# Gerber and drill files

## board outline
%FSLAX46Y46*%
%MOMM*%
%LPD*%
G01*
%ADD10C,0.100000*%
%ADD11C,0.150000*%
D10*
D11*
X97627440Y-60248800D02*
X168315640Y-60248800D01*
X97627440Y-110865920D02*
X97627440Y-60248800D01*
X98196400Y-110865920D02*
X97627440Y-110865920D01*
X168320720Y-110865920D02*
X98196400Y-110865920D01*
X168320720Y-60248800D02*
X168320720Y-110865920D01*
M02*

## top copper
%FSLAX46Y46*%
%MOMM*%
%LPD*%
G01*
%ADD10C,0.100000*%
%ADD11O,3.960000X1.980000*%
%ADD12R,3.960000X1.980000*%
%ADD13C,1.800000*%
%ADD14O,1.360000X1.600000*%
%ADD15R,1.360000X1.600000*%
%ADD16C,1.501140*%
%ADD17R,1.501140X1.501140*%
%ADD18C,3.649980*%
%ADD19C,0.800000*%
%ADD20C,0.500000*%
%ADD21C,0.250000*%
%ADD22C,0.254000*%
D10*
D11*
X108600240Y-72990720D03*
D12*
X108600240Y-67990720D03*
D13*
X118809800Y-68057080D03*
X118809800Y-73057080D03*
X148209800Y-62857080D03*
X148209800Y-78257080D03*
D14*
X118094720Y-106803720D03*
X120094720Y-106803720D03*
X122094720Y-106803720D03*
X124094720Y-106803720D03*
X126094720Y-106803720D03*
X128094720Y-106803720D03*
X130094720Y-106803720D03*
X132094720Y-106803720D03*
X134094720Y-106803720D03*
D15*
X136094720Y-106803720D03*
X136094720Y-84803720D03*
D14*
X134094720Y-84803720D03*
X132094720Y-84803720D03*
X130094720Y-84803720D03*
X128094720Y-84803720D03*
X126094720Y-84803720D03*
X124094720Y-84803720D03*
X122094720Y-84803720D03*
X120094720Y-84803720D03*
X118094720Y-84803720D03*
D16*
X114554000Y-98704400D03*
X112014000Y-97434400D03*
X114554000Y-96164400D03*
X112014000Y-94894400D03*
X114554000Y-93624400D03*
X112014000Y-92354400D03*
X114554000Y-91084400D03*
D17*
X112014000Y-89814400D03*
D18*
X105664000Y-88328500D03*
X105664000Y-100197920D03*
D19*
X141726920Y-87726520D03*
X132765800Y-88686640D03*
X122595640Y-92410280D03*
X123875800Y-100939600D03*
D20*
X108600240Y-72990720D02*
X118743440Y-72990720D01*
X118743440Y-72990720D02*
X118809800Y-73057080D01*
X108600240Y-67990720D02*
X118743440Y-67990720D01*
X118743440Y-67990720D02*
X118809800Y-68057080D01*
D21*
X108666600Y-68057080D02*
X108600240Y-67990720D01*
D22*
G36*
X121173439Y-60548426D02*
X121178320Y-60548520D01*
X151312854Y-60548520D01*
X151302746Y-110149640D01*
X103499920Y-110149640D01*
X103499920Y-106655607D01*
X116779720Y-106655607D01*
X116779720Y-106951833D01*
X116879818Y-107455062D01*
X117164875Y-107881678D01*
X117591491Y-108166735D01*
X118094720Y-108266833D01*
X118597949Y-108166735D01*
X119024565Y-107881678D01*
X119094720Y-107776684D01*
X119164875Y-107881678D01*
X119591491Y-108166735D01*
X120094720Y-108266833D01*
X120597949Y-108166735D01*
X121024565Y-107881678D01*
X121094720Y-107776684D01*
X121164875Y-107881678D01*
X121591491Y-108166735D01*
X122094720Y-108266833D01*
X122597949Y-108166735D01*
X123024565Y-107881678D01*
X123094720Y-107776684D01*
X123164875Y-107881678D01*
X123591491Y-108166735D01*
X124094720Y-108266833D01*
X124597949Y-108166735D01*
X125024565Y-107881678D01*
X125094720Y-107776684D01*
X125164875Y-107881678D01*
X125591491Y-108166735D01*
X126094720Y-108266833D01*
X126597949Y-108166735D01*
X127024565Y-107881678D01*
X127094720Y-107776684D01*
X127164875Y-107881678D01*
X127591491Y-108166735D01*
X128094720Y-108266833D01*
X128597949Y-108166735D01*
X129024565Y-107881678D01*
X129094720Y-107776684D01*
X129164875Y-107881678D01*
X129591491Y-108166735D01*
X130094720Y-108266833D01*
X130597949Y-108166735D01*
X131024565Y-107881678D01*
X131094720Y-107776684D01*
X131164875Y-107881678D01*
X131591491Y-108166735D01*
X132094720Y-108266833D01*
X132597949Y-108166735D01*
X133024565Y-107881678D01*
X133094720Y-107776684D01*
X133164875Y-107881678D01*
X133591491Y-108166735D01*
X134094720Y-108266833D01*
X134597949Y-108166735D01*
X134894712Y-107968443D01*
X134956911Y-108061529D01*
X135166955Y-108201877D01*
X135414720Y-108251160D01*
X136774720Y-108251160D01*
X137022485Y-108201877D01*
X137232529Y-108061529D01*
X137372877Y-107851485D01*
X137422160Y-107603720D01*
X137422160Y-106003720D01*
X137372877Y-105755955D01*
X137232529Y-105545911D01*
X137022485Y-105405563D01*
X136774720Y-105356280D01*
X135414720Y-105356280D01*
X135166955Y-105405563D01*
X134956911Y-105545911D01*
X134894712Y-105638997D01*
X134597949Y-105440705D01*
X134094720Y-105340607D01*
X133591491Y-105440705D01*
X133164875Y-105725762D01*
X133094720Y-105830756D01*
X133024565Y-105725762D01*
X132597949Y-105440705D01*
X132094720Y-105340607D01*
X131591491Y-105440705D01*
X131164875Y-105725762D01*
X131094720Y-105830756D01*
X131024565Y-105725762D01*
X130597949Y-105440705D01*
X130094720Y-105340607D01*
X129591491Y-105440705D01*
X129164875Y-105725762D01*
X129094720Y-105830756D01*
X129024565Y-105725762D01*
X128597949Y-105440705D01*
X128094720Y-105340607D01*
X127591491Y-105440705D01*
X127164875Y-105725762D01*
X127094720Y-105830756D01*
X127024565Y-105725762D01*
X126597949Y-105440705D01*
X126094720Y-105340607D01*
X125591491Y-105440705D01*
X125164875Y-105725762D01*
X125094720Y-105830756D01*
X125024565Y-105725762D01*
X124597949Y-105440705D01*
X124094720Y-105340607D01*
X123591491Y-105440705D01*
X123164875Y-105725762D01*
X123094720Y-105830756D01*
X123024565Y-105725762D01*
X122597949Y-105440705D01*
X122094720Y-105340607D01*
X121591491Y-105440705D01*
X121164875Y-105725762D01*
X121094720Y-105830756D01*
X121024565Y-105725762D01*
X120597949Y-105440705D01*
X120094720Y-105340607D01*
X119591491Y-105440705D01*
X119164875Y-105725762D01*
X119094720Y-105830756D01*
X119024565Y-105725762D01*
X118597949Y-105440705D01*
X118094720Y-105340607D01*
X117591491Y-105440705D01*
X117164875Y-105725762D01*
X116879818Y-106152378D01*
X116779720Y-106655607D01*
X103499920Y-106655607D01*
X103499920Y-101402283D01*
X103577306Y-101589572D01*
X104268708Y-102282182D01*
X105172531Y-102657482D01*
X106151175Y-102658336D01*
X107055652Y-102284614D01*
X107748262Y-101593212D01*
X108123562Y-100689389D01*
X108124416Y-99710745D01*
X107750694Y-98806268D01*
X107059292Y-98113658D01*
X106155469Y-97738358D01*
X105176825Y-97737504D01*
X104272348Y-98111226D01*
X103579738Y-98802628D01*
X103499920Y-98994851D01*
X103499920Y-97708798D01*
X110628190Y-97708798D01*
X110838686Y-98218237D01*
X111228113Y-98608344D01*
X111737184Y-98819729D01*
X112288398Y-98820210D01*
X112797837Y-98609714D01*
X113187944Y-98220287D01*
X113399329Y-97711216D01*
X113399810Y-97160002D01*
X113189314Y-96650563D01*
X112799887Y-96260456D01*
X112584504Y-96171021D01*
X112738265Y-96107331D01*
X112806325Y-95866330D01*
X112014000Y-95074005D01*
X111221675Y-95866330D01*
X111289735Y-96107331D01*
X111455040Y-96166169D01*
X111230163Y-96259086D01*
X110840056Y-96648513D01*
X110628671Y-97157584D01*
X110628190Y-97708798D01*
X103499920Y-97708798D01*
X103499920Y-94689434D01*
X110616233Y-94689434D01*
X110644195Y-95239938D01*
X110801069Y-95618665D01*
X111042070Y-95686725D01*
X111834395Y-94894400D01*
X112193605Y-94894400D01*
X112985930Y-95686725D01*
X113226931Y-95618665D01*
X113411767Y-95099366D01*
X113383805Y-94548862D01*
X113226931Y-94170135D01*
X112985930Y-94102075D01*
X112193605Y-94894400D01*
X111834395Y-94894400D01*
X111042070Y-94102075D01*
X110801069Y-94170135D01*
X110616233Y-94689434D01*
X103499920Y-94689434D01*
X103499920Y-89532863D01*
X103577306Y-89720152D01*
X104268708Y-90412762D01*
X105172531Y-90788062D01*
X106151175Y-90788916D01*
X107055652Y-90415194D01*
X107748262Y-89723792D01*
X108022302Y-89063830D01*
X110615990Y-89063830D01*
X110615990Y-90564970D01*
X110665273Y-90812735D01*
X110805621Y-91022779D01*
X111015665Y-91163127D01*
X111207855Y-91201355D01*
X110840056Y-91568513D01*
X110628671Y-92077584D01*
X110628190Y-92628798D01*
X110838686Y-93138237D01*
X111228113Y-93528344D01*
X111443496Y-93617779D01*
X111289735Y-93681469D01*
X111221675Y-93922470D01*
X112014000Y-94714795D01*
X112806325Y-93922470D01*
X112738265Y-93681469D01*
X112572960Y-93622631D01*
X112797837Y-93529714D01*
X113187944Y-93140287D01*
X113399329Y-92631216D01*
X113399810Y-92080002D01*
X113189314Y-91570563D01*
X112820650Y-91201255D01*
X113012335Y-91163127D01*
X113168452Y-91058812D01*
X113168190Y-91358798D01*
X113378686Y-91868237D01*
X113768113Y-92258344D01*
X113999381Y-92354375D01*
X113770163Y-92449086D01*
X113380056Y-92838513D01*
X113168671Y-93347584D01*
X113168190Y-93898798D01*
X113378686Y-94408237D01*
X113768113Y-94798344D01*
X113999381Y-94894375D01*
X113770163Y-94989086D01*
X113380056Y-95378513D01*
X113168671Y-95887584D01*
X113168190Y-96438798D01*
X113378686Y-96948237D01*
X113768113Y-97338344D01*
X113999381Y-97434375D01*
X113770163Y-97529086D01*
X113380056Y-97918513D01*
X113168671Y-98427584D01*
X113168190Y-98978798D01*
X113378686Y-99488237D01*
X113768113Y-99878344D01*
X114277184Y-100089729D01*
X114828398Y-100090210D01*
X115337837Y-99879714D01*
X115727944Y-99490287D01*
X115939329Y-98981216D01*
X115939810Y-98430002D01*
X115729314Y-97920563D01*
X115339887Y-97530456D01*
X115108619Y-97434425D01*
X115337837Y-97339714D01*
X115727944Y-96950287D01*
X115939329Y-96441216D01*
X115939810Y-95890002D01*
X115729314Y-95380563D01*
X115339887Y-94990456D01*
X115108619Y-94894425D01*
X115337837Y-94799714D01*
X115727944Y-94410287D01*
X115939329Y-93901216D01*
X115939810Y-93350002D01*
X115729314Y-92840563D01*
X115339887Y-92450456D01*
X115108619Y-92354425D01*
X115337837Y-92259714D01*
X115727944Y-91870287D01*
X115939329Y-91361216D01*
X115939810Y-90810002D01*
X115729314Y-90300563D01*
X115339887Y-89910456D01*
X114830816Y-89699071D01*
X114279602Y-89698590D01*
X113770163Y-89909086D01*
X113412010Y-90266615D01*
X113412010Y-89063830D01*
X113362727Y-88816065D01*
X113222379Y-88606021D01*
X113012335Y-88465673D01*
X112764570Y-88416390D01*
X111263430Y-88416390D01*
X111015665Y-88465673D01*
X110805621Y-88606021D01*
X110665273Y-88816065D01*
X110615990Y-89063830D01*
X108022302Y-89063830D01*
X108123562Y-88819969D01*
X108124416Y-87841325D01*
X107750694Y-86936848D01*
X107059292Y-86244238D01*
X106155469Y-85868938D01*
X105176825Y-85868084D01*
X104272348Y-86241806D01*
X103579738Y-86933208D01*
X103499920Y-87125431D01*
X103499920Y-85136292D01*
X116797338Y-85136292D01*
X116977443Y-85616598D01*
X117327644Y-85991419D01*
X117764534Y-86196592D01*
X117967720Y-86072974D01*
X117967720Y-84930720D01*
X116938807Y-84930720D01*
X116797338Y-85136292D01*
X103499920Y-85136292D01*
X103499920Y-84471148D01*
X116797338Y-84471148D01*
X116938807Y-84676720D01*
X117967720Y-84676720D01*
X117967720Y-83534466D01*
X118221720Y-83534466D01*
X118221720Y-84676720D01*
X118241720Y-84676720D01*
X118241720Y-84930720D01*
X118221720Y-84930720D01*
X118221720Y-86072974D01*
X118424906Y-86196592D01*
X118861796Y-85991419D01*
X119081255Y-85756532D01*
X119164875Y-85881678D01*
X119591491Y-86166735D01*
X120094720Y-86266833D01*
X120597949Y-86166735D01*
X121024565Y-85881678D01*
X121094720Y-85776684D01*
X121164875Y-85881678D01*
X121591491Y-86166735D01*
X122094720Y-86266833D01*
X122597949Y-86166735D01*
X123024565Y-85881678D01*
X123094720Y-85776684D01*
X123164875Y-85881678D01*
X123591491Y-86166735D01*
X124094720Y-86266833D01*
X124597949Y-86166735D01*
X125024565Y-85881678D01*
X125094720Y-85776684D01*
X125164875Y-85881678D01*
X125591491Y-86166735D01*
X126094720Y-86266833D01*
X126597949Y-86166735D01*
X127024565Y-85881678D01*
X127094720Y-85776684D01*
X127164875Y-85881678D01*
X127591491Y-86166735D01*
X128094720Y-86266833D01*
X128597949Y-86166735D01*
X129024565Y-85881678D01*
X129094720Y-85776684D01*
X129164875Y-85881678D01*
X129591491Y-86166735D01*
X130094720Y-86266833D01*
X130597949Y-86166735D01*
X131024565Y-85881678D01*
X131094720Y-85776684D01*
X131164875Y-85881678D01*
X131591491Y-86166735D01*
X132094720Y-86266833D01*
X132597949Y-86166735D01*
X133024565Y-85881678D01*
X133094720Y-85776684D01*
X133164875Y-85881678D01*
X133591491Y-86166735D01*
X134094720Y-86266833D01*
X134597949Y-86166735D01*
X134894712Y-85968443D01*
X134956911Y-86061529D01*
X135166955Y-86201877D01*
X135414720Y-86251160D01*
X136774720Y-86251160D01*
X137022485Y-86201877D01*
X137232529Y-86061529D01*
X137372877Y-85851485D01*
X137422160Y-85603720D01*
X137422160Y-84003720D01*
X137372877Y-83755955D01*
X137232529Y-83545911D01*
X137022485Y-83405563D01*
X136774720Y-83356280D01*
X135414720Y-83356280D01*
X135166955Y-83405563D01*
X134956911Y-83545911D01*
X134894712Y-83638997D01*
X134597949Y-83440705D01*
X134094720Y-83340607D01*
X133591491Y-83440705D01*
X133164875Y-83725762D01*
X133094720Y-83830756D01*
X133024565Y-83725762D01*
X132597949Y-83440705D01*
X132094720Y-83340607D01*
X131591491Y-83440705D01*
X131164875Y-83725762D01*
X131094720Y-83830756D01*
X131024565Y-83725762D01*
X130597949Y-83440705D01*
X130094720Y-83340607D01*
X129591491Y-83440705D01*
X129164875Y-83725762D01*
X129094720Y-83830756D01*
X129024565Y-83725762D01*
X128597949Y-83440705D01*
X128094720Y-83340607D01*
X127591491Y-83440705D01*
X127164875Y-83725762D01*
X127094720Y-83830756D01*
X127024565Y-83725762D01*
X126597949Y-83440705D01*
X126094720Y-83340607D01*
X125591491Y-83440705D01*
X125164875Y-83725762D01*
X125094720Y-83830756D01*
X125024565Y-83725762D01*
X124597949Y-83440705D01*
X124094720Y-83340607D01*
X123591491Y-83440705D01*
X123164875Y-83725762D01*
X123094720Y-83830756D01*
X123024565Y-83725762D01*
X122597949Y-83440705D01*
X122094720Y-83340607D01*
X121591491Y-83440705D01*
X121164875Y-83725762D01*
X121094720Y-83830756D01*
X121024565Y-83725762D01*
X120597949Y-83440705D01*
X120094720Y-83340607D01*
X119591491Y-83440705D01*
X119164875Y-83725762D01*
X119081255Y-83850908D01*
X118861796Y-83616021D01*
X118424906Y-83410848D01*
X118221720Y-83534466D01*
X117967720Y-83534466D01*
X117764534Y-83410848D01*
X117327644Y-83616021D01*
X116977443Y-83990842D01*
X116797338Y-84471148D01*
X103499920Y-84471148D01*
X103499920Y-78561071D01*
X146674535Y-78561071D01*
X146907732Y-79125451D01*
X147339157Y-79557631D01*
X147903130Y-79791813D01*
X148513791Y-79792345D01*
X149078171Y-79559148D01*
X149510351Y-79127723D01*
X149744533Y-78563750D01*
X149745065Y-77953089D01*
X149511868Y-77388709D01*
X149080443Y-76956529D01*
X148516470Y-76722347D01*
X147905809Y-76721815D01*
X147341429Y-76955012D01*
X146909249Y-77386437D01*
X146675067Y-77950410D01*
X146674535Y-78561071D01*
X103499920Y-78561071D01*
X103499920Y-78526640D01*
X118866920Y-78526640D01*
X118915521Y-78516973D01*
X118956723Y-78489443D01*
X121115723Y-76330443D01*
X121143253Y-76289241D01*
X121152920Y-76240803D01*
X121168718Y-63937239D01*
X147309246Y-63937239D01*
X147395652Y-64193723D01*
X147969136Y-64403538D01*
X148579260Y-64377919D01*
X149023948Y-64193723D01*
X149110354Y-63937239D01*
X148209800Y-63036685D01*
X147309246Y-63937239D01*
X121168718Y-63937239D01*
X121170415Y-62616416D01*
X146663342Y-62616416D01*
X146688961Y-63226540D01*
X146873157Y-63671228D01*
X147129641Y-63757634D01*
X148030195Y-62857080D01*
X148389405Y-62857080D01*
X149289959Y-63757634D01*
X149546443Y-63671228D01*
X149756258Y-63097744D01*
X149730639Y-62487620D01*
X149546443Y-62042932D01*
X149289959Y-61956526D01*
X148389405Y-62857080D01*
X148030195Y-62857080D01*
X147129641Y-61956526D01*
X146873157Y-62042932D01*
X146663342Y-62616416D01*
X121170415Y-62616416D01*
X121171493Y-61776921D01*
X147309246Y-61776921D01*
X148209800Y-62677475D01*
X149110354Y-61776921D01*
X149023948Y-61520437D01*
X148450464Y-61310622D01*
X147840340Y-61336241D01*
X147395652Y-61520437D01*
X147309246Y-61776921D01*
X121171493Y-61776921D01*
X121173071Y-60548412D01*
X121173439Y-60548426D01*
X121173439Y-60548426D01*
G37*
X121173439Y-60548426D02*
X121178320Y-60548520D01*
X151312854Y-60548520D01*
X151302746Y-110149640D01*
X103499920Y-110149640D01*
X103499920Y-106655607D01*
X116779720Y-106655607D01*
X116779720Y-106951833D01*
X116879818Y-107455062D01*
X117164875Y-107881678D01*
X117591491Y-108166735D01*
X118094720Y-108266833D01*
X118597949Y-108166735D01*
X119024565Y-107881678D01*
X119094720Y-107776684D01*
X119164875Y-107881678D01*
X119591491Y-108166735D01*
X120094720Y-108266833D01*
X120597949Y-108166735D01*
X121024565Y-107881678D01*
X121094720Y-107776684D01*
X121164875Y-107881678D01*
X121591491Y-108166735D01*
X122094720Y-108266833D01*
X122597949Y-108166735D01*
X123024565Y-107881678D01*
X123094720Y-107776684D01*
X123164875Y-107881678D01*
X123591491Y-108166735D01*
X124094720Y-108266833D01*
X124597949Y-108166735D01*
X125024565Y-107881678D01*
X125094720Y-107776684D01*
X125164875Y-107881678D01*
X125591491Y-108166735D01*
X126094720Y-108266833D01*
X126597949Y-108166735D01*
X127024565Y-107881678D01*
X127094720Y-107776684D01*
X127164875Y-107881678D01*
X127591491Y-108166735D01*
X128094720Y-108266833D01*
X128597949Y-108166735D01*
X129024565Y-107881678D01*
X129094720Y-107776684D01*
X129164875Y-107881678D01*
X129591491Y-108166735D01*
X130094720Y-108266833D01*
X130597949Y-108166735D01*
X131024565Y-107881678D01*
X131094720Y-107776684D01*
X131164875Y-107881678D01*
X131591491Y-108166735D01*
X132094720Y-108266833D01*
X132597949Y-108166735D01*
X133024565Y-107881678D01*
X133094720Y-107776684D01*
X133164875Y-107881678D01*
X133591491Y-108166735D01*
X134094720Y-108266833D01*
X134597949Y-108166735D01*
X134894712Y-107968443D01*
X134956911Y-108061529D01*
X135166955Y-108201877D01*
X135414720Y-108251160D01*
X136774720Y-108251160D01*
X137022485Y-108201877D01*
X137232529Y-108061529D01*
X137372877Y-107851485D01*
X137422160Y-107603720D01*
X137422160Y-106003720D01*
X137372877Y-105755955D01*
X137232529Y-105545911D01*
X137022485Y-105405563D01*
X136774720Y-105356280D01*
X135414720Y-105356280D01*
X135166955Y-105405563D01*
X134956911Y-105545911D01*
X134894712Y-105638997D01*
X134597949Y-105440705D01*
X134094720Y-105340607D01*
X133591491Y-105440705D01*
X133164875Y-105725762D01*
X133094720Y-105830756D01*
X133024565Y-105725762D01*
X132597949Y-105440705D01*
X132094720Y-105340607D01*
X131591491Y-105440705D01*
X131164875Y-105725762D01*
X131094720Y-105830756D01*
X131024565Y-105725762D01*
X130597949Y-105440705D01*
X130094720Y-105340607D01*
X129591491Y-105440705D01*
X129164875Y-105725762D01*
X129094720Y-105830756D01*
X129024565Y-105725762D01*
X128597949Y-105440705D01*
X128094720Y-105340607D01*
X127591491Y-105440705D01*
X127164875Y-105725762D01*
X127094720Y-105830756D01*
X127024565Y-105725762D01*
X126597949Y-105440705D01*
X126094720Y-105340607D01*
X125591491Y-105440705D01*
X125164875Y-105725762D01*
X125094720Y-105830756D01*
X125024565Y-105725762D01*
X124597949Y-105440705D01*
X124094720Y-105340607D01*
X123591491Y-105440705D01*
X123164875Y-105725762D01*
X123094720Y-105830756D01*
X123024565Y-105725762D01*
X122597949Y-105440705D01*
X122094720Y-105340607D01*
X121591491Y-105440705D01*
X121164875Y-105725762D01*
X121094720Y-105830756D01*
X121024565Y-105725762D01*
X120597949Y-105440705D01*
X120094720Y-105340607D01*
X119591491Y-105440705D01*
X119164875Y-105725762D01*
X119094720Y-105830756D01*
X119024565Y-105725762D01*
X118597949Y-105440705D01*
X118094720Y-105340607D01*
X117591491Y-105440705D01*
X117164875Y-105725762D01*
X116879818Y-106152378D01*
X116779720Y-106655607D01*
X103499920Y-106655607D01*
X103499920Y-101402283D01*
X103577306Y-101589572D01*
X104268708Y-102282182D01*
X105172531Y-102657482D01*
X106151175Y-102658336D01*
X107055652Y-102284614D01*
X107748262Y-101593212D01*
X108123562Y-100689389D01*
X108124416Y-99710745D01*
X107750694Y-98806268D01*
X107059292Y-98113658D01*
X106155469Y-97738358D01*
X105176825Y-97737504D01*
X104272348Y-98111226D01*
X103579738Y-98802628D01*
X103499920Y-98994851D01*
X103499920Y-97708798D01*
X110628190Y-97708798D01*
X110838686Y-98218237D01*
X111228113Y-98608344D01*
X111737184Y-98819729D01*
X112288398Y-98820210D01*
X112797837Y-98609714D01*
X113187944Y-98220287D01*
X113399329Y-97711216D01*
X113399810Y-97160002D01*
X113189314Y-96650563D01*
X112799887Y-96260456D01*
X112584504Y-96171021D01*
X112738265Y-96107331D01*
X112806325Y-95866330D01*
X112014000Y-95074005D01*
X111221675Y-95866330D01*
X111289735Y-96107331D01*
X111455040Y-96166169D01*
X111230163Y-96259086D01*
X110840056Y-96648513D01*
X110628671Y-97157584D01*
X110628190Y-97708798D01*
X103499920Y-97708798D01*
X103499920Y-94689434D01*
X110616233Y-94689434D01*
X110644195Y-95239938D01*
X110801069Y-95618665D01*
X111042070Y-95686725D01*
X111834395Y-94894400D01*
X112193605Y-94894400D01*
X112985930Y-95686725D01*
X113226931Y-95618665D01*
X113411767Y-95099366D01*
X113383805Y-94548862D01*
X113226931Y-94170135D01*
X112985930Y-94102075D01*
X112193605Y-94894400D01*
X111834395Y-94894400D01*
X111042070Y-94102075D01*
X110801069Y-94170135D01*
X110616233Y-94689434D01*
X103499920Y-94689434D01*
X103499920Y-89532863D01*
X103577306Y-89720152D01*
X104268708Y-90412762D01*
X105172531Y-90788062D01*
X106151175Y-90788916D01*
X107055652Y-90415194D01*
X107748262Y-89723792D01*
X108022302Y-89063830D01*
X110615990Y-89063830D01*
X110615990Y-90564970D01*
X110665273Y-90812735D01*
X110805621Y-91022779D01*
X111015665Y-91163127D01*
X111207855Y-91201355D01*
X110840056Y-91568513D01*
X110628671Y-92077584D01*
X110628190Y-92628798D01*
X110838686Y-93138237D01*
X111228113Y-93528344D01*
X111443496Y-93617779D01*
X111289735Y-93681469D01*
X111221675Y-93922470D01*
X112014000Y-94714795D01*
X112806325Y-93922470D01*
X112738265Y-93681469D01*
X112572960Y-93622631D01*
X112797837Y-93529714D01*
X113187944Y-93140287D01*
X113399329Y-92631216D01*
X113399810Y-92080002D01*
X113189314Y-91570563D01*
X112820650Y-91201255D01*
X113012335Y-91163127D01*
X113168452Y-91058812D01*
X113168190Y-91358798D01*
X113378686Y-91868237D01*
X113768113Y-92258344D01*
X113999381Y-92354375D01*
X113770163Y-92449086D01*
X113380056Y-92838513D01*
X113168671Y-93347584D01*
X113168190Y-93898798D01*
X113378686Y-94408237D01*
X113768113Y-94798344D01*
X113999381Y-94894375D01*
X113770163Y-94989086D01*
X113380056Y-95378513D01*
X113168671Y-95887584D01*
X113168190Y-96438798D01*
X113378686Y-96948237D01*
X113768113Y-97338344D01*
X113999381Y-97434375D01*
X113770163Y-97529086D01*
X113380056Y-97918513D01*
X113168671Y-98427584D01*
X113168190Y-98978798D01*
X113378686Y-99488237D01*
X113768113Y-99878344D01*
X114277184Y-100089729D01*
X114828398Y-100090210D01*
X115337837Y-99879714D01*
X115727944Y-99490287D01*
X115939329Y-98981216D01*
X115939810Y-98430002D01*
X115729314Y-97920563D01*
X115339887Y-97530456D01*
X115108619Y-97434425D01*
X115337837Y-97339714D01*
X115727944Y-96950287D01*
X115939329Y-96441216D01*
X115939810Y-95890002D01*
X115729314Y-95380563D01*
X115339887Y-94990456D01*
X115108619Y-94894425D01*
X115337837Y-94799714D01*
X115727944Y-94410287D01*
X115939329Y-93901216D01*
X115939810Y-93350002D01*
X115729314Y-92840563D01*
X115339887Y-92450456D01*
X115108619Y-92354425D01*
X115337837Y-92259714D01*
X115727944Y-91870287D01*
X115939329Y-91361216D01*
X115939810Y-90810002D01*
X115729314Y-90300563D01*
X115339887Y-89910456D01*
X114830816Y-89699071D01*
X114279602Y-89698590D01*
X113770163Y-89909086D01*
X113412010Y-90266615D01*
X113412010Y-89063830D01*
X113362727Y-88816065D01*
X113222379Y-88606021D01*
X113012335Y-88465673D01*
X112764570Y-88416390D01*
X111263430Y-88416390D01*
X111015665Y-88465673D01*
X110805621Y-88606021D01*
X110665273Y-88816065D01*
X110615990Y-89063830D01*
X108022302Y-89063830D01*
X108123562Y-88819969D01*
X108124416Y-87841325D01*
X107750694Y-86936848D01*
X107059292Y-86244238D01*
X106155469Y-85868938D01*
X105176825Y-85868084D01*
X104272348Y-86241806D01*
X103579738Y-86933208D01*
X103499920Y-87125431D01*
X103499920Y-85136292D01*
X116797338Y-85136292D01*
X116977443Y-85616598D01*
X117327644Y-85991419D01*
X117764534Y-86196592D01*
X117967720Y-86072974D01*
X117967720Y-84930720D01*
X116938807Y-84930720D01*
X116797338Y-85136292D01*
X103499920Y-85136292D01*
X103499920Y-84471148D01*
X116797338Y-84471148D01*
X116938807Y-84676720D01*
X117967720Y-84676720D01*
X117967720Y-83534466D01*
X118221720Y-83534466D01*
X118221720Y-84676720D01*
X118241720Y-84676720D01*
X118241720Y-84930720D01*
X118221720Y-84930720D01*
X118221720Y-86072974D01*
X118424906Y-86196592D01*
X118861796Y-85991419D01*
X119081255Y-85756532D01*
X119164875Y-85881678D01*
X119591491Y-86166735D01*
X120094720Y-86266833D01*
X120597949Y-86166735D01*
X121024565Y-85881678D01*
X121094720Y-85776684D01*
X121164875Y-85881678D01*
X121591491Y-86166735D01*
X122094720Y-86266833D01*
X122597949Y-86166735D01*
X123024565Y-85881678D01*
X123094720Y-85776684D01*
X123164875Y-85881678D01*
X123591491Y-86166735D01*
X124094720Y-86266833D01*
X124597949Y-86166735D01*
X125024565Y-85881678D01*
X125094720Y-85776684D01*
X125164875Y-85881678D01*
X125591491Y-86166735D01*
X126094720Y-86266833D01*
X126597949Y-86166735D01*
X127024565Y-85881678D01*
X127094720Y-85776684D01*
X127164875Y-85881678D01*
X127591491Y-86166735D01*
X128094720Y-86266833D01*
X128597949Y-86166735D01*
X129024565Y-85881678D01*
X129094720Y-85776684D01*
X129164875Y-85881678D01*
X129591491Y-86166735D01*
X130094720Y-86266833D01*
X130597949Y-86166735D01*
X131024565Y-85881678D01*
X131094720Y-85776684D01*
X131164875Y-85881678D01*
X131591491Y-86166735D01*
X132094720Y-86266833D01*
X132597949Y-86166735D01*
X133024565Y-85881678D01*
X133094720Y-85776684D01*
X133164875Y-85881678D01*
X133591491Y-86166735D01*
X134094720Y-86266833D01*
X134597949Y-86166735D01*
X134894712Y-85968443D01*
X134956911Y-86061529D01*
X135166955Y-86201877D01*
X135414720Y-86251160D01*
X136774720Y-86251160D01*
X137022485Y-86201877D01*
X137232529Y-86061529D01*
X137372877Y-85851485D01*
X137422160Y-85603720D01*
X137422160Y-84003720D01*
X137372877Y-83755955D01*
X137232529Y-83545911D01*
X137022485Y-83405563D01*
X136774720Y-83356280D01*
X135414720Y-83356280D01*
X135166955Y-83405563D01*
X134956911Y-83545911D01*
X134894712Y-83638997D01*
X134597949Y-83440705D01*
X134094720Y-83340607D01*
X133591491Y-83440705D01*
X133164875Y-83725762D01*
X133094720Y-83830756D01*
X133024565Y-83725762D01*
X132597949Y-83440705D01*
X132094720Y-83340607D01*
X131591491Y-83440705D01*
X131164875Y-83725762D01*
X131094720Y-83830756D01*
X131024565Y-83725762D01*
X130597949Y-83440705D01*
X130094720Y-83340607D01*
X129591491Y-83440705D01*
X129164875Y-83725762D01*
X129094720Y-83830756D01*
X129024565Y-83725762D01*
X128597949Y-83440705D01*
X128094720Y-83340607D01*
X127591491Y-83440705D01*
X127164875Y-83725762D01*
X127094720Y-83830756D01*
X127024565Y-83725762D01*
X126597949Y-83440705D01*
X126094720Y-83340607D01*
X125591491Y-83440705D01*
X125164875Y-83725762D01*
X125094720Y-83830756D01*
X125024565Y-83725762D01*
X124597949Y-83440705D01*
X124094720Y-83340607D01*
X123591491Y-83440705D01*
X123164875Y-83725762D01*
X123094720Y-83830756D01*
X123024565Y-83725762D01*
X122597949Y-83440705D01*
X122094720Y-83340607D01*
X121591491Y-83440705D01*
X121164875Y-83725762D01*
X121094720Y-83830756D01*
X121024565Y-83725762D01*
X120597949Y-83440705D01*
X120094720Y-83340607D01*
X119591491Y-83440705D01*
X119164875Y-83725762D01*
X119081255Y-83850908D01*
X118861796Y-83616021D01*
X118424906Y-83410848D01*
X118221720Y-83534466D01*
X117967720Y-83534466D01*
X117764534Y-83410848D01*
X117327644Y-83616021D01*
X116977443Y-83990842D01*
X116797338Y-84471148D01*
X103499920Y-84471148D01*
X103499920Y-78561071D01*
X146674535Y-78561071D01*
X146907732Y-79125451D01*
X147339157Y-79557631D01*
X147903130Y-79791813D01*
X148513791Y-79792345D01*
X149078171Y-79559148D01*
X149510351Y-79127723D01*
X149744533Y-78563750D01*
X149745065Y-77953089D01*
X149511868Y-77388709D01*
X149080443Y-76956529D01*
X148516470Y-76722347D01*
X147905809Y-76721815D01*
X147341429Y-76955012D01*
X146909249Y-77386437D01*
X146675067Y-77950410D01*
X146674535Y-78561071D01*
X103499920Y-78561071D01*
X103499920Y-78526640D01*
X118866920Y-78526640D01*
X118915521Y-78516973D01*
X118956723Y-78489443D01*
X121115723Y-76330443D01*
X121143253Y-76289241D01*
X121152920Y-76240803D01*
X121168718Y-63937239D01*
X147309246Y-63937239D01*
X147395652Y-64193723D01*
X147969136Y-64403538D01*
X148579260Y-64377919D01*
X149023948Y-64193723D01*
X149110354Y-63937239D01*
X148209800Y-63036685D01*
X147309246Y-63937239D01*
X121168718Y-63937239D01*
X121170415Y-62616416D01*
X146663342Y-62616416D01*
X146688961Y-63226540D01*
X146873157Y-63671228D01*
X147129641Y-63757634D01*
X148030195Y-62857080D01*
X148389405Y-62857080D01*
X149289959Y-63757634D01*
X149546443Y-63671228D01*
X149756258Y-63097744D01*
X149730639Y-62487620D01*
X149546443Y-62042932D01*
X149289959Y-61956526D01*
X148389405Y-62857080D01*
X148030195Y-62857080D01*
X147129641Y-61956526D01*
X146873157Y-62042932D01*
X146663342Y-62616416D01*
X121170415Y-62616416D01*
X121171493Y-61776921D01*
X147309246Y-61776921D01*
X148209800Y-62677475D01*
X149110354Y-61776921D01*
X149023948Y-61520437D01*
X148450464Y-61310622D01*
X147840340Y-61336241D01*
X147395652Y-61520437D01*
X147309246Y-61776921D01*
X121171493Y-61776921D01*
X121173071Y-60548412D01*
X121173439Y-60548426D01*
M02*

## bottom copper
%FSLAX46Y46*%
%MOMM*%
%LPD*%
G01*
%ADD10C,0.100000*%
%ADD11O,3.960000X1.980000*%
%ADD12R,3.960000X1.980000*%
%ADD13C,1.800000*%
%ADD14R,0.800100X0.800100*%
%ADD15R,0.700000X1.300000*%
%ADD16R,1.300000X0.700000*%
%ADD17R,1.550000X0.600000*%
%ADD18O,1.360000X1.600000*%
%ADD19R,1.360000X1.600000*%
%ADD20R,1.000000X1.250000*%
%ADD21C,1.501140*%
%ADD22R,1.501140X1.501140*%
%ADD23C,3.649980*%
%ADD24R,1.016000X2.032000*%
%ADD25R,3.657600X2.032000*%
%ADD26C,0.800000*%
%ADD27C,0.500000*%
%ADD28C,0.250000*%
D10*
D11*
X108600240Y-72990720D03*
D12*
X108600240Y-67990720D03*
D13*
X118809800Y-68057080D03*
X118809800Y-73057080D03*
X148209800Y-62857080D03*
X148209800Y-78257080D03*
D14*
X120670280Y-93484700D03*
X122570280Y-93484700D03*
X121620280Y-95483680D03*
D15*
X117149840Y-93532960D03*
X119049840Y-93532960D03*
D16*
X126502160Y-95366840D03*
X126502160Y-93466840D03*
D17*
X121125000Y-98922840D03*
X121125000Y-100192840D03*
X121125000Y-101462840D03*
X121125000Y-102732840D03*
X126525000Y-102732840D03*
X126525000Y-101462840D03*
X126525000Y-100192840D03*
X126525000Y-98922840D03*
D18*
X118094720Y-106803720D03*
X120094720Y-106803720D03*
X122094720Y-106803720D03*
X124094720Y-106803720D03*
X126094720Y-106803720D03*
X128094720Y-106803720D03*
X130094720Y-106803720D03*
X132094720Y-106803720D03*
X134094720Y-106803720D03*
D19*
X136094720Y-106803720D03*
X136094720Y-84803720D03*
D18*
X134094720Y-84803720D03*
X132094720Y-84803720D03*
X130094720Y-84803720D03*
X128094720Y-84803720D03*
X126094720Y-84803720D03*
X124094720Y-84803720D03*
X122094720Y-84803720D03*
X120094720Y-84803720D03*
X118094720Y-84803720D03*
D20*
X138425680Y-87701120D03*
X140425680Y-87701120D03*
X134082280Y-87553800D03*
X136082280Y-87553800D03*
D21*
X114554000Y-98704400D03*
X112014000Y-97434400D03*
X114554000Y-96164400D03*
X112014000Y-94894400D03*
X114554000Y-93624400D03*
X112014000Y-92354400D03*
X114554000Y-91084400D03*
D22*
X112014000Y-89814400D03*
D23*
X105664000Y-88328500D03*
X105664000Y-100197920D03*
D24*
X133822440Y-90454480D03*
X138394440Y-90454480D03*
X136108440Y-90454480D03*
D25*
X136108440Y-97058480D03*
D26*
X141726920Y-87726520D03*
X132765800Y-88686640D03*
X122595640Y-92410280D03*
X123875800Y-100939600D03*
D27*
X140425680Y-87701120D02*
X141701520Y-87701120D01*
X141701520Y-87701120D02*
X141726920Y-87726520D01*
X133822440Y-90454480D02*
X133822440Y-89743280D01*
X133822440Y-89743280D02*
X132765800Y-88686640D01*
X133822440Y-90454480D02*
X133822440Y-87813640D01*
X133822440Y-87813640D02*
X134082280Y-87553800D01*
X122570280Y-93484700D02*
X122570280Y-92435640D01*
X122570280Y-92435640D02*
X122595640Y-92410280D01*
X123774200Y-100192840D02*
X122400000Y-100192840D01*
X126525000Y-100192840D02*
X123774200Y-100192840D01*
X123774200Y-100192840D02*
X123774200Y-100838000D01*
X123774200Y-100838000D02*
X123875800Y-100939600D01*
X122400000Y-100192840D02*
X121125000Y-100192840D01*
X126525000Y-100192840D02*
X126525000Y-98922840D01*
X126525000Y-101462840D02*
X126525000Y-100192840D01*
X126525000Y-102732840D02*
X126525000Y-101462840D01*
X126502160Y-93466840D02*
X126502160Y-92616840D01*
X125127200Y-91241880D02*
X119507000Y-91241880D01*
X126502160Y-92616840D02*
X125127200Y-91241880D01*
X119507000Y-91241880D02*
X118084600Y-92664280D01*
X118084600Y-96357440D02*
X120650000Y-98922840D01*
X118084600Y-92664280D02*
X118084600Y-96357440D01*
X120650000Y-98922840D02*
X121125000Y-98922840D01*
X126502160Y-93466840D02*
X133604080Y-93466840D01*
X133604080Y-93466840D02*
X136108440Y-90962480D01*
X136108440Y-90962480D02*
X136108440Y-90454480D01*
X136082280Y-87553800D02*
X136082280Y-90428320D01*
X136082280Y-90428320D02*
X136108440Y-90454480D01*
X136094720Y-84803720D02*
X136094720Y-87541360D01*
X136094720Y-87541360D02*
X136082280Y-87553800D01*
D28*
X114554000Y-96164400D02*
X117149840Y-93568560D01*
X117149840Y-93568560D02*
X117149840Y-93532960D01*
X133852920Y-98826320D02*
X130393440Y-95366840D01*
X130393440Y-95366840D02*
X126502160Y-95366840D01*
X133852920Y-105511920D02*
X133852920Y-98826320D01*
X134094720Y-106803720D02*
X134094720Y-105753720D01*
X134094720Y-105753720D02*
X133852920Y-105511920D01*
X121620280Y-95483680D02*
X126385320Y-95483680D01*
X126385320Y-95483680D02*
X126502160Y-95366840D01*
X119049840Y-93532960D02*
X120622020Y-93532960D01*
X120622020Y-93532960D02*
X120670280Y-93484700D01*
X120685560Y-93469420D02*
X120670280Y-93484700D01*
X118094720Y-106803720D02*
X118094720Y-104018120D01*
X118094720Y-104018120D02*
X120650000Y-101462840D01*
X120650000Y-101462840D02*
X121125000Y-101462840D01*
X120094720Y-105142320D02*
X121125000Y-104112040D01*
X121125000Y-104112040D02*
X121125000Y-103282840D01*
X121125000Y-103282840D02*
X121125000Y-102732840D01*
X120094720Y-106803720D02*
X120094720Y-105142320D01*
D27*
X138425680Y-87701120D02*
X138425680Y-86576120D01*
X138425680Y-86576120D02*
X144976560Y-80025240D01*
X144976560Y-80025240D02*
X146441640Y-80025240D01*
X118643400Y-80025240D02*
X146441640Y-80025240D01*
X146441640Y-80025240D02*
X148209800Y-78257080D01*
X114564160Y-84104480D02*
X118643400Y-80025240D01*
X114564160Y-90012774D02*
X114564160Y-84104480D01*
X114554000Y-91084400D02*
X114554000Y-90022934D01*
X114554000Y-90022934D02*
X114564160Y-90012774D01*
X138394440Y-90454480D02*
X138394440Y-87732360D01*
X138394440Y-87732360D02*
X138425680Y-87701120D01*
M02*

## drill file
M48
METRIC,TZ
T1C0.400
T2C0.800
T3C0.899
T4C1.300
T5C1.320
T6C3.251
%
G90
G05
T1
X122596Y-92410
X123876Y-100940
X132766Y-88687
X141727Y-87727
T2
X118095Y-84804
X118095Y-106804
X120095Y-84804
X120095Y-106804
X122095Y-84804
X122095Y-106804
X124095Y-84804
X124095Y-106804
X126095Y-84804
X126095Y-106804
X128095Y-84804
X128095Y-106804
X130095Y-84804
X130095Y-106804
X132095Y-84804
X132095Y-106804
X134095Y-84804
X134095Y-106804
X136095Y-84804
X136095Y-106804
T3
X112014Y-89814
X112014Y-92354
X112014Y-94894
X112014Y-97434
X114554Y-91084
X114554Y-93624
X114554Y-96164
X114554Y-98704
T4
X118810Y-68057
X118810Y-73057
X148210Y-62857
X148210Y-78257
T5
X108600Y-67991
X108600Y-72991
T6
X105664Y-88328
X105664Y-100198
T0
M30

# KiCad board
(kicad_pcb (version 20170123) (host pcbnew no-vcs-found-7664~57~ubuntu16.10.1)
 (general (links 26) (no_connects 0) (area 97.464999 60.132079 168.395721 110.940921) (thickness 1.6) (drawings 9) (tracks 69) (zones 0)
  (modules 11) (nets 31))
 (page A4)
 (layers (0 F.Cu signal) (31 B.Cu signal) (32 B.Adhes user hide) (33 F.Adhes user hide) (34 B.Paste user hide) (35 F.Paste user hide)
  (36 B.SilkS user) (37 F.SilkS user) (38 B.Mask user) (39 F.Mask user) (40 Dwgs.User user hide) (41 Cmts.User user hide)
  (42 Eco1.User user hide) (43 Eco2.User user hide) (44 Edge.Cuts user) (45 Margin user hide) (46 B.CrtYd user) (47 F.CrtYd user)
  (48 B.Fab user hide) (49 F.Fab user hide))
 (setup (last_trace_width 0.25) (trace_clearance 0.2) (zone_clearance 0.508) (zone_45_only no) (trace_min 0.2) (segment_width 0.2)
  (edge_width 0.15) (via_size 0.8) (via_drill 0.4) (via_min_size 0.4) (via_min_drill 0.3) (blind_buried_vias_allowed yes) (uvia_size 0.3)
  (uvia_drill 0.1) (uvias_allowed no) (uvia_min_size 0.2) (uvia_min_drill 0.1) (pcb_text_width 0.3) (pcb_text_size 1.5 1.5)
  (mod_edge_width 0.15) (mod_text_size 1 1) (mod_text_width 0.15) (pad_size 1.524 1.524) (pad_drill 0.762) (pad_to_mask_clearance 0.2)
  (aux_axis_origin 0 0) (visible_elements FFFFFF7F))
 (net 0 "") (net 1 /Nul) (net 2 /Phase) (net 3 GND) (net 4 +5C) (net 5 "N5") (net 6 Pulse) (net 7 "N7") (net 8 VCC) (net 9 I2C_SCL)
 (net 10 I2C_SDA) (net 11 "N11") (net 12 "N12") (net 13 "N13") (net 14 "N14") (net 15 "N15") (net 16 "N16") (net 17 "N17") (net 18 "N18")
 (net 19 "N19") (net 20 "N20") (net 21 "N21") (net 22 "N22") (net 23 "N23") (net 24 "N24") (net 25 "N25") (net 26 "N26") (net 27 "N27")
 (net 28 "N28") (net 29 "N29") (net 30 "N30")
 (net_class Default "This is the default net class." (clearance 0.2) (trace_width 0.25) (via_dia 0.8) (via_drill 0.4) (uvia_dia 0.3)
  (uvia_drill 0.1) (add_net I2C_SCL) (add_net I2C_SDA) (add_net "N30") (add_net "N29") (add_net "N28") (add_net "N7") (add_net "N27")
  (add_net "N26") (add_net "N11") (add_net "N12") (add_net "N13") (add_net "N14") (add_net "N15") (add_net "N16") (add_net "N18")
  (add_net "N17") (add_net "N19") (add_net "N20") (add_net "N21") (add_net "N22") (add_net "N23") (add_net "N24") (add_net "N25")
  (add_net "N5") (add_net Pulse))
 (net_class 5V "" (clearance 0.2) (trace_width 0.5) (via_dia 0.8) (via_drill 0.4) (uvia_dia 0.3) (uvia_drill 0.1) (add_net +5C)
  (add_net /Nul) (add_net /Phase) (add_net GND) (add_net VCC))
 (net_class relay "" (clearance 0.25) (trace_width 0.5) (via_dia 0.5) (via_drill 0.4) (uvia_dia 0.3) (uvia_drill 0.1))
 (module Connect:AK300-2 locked (layer F.Cu) (at 108.60024 67.99072 270)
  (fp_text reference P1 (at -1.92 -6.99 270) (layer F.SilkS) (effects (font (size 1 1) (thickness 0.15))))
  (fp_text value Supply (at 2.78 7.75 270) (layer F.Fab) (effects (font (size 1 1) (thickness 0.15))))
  (pad 2 thru_hole oval (at 5 0 270) (size 1.98 3.96) (drill 1.32) (layers *.Cu F.Paste F.Mask) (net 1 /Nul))
  (pad 1 thru_hole rect (at 0 0 270) (size 1.98 3.96) (drill 1.32) (layers *.Cu F.Paste F.Mask) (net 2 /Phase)))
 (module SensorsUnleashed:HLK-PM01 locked (layer F.Cu) (at 133.0198 70.61708)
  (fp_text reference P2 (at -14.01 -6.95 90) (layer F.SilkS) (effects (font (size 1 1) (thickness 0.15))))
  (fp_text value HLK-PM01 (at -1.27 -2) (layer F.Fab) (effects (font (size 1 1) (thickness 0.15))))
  (pad 1 thru_hole circle (at -14.21 -2.56) (size 1.8 1.8) (drill 1.3) (layers *.Cu *.Mask F.SilkS) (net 2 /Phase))
  (pad 2 thru_hole circle (at -14.21 2.44) (size 1.8 1.8) (drill 1.3) (layers *.Cu *.Mask F.SilkS) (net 1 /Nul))
  (pad 3 thru_hole circle (at 15.19 -7.76) (size 1.8 1.8) (drill 1.3) (layers *.Cu *.Mask F.SilkS) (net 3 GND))
  (pad 4 thru_hole circle (at 15.19 7.64) (size 1.8 1.8) (drill 1.3) (layers *.Cu *.Mask F.SilkS) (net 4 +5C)))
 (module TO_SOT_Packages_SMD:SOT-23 (layer B.Cu) (at 121.62028 94.48546)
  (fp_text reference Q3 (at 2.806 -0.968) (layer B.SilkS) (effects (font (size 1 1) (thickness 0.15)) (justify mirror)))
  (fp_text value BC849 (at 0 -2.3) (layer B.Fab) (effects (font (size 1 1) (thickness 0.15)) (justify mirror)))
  (pad 1 smd rect (at -0.95 -1.00076) (size 0.8001 0.8001) (layers B.Cu B.Paste B.Mask) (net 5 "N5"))
  (pad 2 smd rect (at 0.95 -1.00076) (size 0.8001 0.8001) (layers B.Cu B.Paste B.Mask) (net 3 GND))
  (pad 3 smd rect (at 0 0.99822) (size 0.8001 0.8001) (layers B.Cu B.Paste B.Mask) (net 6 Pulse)))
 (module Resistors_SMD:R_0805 (layer B.Cu) (at 118.09984 93.53296)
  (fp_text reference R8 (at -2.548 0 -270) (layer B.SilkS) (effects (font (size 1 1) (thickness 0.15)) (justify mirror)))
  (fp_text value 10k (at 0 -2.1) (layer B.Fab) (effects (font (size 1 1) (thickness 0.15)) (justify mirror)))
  (pad 1 smd rect (at -0.95 0) (size 0.7 1.3) (layers B.Cu B.Paste B.Mask) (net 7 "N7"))
  (pad 2 smd rect (at 0.95 0) (size 0.7 1.3) (layers B.Cu B.Paste B.Mask) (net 5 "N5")))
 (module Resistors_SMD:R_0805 (layer B.Cu) (at 126.50216 94.41684 270)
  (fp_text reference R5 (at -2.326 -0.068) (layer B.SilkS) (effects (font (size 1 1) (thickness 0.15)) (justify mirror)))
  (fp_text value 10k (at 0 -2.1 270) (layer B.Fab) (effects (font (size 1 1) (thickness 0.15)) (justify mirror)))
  (pad 2 smd rect (at 0.95 0 270) (size 0.7 1.3) (layers B.Cu B.Paste B.Mask) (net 6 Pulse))
  (pad 1 smd rect (at -0.95 0 270) (size 0.7 1.3) (layers B.Cu B.Paste B.Mask) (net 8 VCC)))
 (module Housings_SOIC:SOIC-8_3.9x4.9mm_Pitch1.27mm (layer B.Cu) (at 123.825 100.82784 180)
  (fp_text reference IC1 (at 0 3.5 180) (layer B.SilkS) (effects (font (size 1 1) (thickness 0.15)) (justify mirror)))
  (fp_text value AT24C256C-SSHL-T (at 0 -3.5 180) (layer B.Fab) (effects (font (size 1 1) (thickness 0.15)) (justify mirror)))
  (pad 8 smd rect (at 2.7 1.905 180) (size 1.55 0.6) (layers B.Cu B.Paste B.Mask) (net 8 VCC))
  (pad 7 smd rect (at 2.7 0.635 180) (size 1.55 0.6) (layers B.Cu B.Paste B.Mask) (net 3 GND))
  (pad 6 smd rect (at 2.7 -0.635 180) (size 1.55 0.6) (layers B.Cu B.Paste B.Mask) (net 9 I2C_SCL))
  (pad 5 smd rect (at 2.7 -1.905 180) (size 1.55 0.6) (layers B.Cu B.Paste B.Mask) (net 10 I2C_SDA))
  (pad 4 smd rect (at -2.7 -1.905 180) (size 1.55 0.6) (layers B.Cu B.Paste B.Mask) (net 3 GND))
  (pad 3 smd rect (at -2.7 -0.635 180) (size 1.55 0.6) (layers B.Cu B.Paste B.Mask) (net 3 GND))
  (pad 2 smd rect (at -2.7 0.635 180) (size 1.55 0.6) (layers B.Cu B.Paste B.Mask) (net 3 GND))
  (pad 1 smd rect (at -2.7 1.905 180) (size 1.55 0.6) (layers B.Cu B.Paste B.Mask) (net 3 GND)))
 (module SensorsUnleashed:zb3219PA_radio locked (layer F.Cu) (at 127.29972 95.80372 270)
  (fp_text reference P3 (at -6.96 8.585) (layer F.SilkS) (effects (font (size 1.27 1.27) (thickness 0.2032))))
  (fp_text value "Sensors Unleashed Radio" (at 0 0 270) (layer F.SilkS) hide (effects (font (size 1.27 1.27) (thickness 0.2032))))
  (pad 11 thru_hole oval (at 11 9.205 180) (size 1.36 1.6) (drill 0.8) (layers *.Cu *.Mask F.SilkS) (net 9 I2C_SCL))
  (pad 12 thru_hole oval (at 11 7.205 180) (size 1.36 1.6) (drill 0.8) (layers *.Cu *.Mask F.SilkS) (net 10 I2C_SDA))
  (pad 13 thru_hole oval (at 11 5.205 180) (size 1.36 1.6) (drill 0.8) (layers *.Cu *.Mask F.SilkS) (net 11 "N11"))
  (pad 14 thru_hole oval (at 11 3.205 180) (size 1.36 1.6) (drill 0.8) (layers *.Cu *.Mask F.SilkS) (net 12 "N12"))
  (pad 15 thru_hole oval (at 11 1.205 180) (size 1.36 1.6) (drill 0.8) (layers *.Cu *.Mask F.SilkS) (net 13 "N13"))
  (pad 16 thru_hole oval (at 11 -0.795 180) (size 1.36 1.6) (drill 0.8) (layers *.Cu *.Mask F.SilkS) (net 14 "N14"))
  (pad 17 thru_hole oval (at 11 -2.795 180) (size 1.36 1.6) (drill 0.8) (layers *.Cu *.Mask F.SilkS) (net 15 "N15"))
  (pad 18 thru_hole oval (at 11 -4.795 180) (size 1.36 1.6) (drill 0.8) (layers *.Cu *.Mask F.SilkS) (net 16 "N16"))
  (pad 19 thru_hole oval (at 11 -6.795 180) (size 1.36 1.6) (drill 0.8) (layers *.Cu *.Mask F.SilkS) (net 6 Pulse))
  (pad 20 thru_hole rect (at 11 -8.795 180) (size 1.36 1.6) (drill 0.8) (layers *.Cu *.Mask F.SilkS) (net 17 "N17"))
  (pad 1 thru_hole rect (at -11 -8.795 180) (size 1.36 1.6) (drill 0.8) (layers *.Cu *.Mask F.SilkS) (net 8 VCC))
  (pad 2 thru_hole oval (at -11 -6.795 180) (size 1.36 1.6) (drill 0.8) (layers *.Cu *.Mask F.SilkS) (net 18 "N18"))
  (pad 3 thru_hole oval (at -11 -4.795 180) (size 1.36 1.6) (drill 0.8) (layers *.Cu *.Mask F.SilkS) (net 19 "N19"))
  (pad 4 thru_hole oval (at -11 -2.795 180) (size 1.36 1.6) (drill 0.8) (layers *.Cu *.Mask F.SilkS) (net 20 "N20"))
  (pad 5 thru_hole oval (at -11 -0.795 180) (size 1.36 1.6) (drill 0.8) (layers *.Cu *.Mask F.SilkS) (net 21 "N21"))
  (pad 6 thru_hole oval (at -11 1.205 180) (size 1.36 1.6) (drill 0.8) (layers *.Cu *.Mask F.SilkS) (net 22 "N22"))
  (pad 7 thru_hole oval (at -11 3.205 180) (size 1.36 1.6) (drill 0.8) (layers *.Cu *.Mask F.SilkS) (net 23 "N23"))
  (pad 8 thru_hole oval (at -11 5.205 180) (size 1.36 1.6) (drill 0.8) (layers *.Cu *.Mask F.SilkS) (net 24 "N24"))
  (pad 9 thru_hole oval (at -11 7.205 180) (size 1.36 1.6) (drill 0.8) (layers *.Cu *.Mask F.SilkS) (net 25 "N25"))
  (pad 10 thru_hole oval (at -11 9.205 180) (size 1.36 1.6) (drill 0.8) (layers *.Cu *.Mask F.SilkS) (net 3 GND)))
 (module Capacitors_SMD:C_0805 (layer B.Cu) (at 139.42568 87.70112)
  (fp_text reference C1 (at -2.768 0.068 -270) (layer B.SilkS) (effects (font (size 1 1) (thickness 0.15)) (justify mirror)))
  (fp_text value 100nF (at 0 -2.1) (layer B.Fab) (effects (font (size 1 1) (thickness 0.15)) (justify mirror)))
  (pad 1 smd rect (at -1 0) (size 1 1.25) (layers B.Cu B.Paste B.Mask) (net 4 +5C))
  (pad 2 smd rect (at 1 0) (size 1 1.25) (layers B.Cu B.Paste B.Mask) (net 3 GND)))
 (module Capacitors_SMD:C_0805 (layer B.Cu) (at 135.08228 87.5538 180)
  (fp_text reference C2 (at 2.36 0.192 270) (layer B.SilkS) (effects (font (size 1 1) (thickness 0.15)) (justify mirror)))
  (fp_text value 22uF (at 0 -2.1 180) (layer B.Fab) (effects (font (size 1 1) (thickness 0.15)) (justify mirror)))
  (pad 2 smd rect (at 1 0 180) (size 1 1.25) (layers B.Cu B.Paste B.Mask) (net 3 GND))
  (pad 1 smd rect (at -1 0 180) (size 1 1.25) (layers B.Cu B.Paste B.Mask) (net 8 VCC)))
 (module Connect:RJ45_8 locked (layer F.Cu) (at 105.664 94.2594 270)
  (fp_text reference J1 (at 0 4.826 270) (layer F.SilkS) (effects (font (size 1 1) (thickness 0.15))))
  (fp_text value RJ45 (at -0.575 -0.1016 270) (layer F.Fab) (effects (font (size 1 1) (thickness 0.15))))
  (pad 8 thru_hole circle (at 4.445 -8.89 270) (size 1.50114 1.50114) (drill 0.89916) (layers *.Cu *.Mask) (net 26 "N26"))
  (pad 7 thru_hole circle (at 3.175 -6.35 270) (size 1.50114 1.50114) (drill 0.89916) (layers *.Cu *.Mask) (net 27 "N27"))
  (pad 6 thru_hole circle (at 1.905 -8.89 270) (size 1.50114 1.50114) (drill 0.89916) (layers *.Cu *.Mask) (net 7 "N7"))
  (pad 5 thru_hole circle (at 0.635 -6.35 270) (size 1.50114 1.50114) (drill 0.89916) (layers *.Cu *.Mask) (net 3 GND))
  (pad 4 thru_hole circle (at -0.635 -8.89 270) (size 1.50114 1.50114) (drill 0.89916) (layers *.Cu *.Mask) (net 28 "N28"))
  (pad 3 thru_hole circle (at -1.905 -6.35 270) (size 1.50114 1.50114) (drill 0.89916) (layers *.Cu *.Mask) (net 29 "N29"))
  (pad 2 thru_hole circle (at -3.175 -8.89 270) (size 1.50114 1.50114) (drill 0.89916) (layers *.Cu *.Mask) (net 4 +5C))
  (pad 1 thru_hole rect (at -4.445 -6.35 270) (size 1.50114 1.50114) (drill 0.89916) (layers *.Cu *.Mask) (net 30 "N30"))
  (pad Hole np_thru_hole circle (at -5.9309 0 270) (size 3.64998 3.64998) (drill 3.2512) (layers *.Cu *.SilkS *.Mask))
  (pad Hole np_thru_hole circle (at 5.93852 0 270) (size 3.64998 3.64998) (drill 3.2512) (layers *.Cu *.SilkS *.Mask)))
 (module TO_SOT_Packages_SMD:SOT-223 (layer B.Cu) (at 136.10844 93.75648)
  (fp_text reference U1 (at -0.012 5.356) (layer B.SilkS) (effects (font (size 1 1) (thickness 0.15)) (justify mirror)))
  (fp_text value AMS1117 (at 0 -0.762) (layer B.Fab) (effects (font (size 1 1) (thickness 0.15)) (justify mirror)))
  (pad 1 smd rect (at -2.286 -3.302) (size 1.016 2.032) (layers B.Cu B.Paste B.Mask) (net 3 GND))
  (pad 3 smd rect (at 2.286 -3.302) (size 1.016 2.032) (layers B.Cu B.Paste B.Mask) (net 4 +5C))
  (pad 2 smd rect (at 0 -3.302) (size 1.016 2.032) (layers B.Cu B.Paste B.Mask) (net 8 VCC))
  (pad 4 smd rect (at 0 3.302) (size 3.6576 2.032) (layers B.Cu B.Paste B.Mask)))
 (gr_line (start 97.62744 60.2488) (end 168.31564 60.2488) (layer Edge.Cuts) (width 0.15))
 (gr_line (start 97.62744 110.86592) (end 97.62744 60.2488) (layer Edge.Cuts) (width 0.15))
 (gr_line (start 98.1964 110.86592) (end 97.62744 110.86592) (layer Edge.Cuts) (width 0.15))
 (gr_line (start 168.32072 110.86592) (end 98.1964 110.86592) (layer Edge.Cuts) (width 0.15))
 (gr_line (start 168.32072 60.2488) (end 168.32072 110.86592) (layer Edge.Cuts) (width 0.15))
 (segment (start 140.42568 87.70112) (end 141.70152 87.70112) (width 0.5) (layer B.Cu) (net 3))
 (segment (start 141.70152 87.70112) (end 141.72692 87.72652) (width 0.5) (layer B.Cu) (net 3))
 (via (at 141.72692 87.72652) (size 0.8) (drill 0.4) (layers F.Cu B.Cu) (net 3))
 (segment (start 133.82244 90.45448) (end 133.82244 89.74328) (width 0.5) (layer B.Cu) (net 3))
 (segment (start 133.82244 89.74328) (end 132.7658 88.68664) (width 0.5) (layer B.Cu) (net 3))
 (via (at 132.7658 88.68664) (size 0.8) (drill 0.4) (layers F.Cu B.Cu) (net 3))
 (segment (start 133.82244 90.45448) (end 133.82244 87.81364) (width 0.5) (layer B.Cu) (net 3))
 (segment (start 133.82244 87.81364) (end 134.08228 87.5538) (width 0.5) (layer B.Cu) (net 3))
 (segment (start 122.57028 93.4847) (end 122.57028 92.43564) (width 0.5) (layer B.Cu) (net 3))
 (segment (start 122.57028 92.43564) (end 122.59564 92.41028) (width 0.5) (layer B.Cu) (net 3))
 (via (at 122.59564 92.41028) (size 0.8) (drill 0.4) (layers F.Cu B.Cu) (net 3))
 (segment (start 123.7742 100.19284) (end 122.4 100.19284) (width 0.5) (layer B.Cu) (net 3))
 (segment (start 126.525 100.19284) (end 123.7742 100.19284) (width 0.5) (layer B.Cu) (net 3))
 (segment (start 123.7742 100.19284) (end 123.7742 100.838) (width 0.5) (layer B.Cu) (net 3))
 (segment (start 123.7742 100.838) (end 123.8758 100.9396) (width 0.5) (layer B.Cu) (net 3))
 (via (at 123.8758 100.9396) (size 0.8) (drill 0.4) (layers F.Cu B.Cu) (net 3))
 (segment (start 122.4 100.19284) (end 121.125 100.19284) (width 0.5) (layer B.Cu) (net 3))
 (segment (start 126.525 100.19284) (end 126.525 98.92284) (width 0.5) (layer B.Cu) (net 3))
 (segment (start 126.525 101.46284) (end 126.525 100.19284) (width 0.5) (layer B.Cu) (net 3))
 (segment (start 126.525 102.73284) (end 126.525 101.46284) (width 0.5) (layer B.Cu) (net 3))
 (segment (start 126.50216 93.46684) (end 126.50216 92.61684) (width 0.5) (layer B.Cu) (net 8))
 (segment (start 125.1272 91.24188) (end 119.507 91.24188) (width 0.5) (layer B.Cu) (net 8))
 (segment (start 126.50216 92.61684) (end 125.1272 91.24188) (width 0.5) (layer B.Cu) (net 8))
 (segment (start 119.507 91.24188) (end 118.0846 92.66428) (width 0.5) (layer B.Cu) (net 8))
 (segment (start 118.0846 96.35744) (end 120.65 98.92284) (width 0.5) (layer B.Cu) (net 8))
 (segment (start 118.0846 92.66428) (end 118.0846 96.35744) (width 0.5) (layer B.Cu) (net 8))
 (segment (start 120.65 98.92284) (end 121.125 98.92284) (width 0.5) (layer B.Cu) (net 8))
 (segment (start 126.50216 93.46684) (end 133.60408 93.46684) (width 0.5) (layer B.Cu) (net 8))
 (segment (start 133.60408 93.46684) (end 136.10844 90.96248) (width 0.5) (layer B.Cu) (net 8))
 (segment (start 136.10844 90.96248) (end 136.10844 90.45448) (width 0.5) (layer B.Cu) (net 8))
 (segment (start 136.08228 87.5538) (end 136.08228 90.42832) (width 0.5) (layer B.Cu) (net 8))
 (segment (start 136.08228 90.42832) (end 136.10844 90.45448) (width 0.5) (layer B.Cu) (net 8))
 (segment (start 136.09472 84.80372) (end 136.09472 87.54136) (width 0.5) (layer B.Cu) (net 8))
 (segment (start 136.09472 87.54136) (end 136.08228 87.5538) (width 0.5) (layer B.Cu) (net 8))
 (segment (start 114.554 96.1644) (end 117.14984 93.56856) (width 0.25) (layer B.Cu) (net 7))
 (segment (start 117.14984 93.56856) (end 117.14984 93.53296) (width 0.25) (layer B.Cu) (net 7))
 (segment (start 133.85292 98.82632) (end 130.39344 95.36684) (width 0.25) (layer B.Cu) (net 6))
 (segment (start 130.39344 95.36684) (end 126.50216 95.36684) (width 0.25) (layer B.Cu) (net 6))
 (segment (start 133.85292 105.51192) (end 133.85292 98.82632) (width 0.25) (layer B.Cu) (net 6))
 (segment (start 134.09472 106.80372) (end 134.09472 105.75372) (width 0.25) (layer B.Cu) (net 6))
 (segment (start 134.09472 105.75372) (end 133.85292 105.51192) (width 0.25) (layer B.Cu) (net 6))
 (segment (start 121.62028 95.48368) (end 126.38532 95.48368) (width 0.25) (layer B.Cu) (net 6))
 (segment (start 126.38532 95.48368) (end 126.50216 95.36684) (width 0.25) (layer B.Cu) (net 6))
 (segment (start 119.04984 93.53296) (end 120.62202 93.53296) (width 0.25) (layer B.Cu) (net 5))
 (segment (start 120.62202 93.53296) (end 120.67028 93.4847) (width 0.25) (layer B.Cu) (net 5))
 (segment (start 120.68556 93.46942) (end 120.67028 93.4847) (width 0.25) (layer B.Cu) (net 5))
 (segment (start 118.09472 106.80372) (end 118.09472 104.01812) (width 0.25) (layer B.Cu) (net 9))
 (segment (start 118.09472 104.01812) (end 120.65 101.46284) (width 0.25) (layer B.Cu) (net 9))
 (segment (start 120.65 101.46284) (end 121.125 101.46284) (width 0.25) (layer B.Cu) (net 9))
 (segment (start 120.09472 105.14232) (end 121.125 104.11204) (width 0.25) (layer B.Cu) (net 10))
 (segment (start 121.125 104.11204) (end 121.125 103.28284) (width 0.25) (layer B.Cu) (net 10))
 (segment (start 121.125 103.28284) (end 121.125 102.73284) (width 0.25) (layer B.Cu) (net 10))
 (segment (start 120.09472 106.80372) (end 120.09472 105.14232) (width 0.25) (layer B.Cu) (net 10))
 (segment (start 108.60024 72.99072) (end 118.74344 72.99072) (width 0.5) (layer F.Cu) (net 1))
 (segment (start 118.74344 72.99072) (end 118.8098 73.05708) (width 0.5) (layer F.Cu) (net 1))
 (segment (start 108.60024 67.99072) (end 118.74344 67.99072) (width 0.5) (layer F.Cu) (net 2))
 (segment (start 118.74344 67.99072) (end 118.8098 68.05708) (width 0.5) (layer F.Cu) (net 2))
 (segment (start 108.6666 68.05708) (end 108.60024 67.99072) (width 0.25) (layer F.Cu) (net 2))
 (segment (start 138.42568 87.70112) (end 138.42568 86.57612) (width 0.5) (layer B.Cu) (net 4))
 (segment (start 138.42568 86.57612) (end 144.97656 80.02524) (width 0.5) (layer B.Cu) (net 4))
 (segment (start 144.97656 80.02524) (end 146.44164 80.02524) (width 0.5) (layer B.Cu) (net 4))
 (segment (start 118.6434 80.02524) (end 146.44164 80.02524) (width 0.5) (layer B.Cu) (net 4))
 (segment (start 146.44164 80.02524) (end 148.2098 78.25708) (width 0.5) (layer B.Cu) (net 4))
 (segment (start 114.56416 84.10448) (end 118.6434 80.02524) (width 0.5) (layer B.Cu) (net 4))
 (segment (start 114.56416 90.012774) (end 114.56416 84.10448) (width 0.5) (layer B.Cu) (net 4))
 (segment (start 114.554 91.0844) (end 114.554 90.022934) (width 0.5) (layer B.Cu) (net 4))
 (segment (start 114.554 90.022934) (end 114.56416 90.012774) (width 0.5) (layer B.Cu) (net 4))
 (segment (start 138.39444 90.45448) (end 138.39444 87.73236) (width 0.5) (layer B.Cu) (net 4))
 (segment (start 138.39444 87.73236) (end 138.42568 87.70112) (width 0.5) (layer B.Cu) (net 4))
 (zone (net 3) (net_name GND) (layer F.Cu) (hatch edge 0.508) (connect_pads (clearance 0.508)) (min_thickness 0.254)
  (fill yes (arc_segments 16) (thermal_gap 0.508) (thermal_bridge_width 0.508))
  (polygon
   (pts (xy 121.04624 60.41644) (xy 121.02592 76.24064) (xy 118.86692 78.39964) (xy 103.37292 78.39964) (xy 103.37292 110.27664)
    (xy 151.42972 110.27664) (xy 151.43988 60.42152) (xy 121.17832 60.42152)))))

